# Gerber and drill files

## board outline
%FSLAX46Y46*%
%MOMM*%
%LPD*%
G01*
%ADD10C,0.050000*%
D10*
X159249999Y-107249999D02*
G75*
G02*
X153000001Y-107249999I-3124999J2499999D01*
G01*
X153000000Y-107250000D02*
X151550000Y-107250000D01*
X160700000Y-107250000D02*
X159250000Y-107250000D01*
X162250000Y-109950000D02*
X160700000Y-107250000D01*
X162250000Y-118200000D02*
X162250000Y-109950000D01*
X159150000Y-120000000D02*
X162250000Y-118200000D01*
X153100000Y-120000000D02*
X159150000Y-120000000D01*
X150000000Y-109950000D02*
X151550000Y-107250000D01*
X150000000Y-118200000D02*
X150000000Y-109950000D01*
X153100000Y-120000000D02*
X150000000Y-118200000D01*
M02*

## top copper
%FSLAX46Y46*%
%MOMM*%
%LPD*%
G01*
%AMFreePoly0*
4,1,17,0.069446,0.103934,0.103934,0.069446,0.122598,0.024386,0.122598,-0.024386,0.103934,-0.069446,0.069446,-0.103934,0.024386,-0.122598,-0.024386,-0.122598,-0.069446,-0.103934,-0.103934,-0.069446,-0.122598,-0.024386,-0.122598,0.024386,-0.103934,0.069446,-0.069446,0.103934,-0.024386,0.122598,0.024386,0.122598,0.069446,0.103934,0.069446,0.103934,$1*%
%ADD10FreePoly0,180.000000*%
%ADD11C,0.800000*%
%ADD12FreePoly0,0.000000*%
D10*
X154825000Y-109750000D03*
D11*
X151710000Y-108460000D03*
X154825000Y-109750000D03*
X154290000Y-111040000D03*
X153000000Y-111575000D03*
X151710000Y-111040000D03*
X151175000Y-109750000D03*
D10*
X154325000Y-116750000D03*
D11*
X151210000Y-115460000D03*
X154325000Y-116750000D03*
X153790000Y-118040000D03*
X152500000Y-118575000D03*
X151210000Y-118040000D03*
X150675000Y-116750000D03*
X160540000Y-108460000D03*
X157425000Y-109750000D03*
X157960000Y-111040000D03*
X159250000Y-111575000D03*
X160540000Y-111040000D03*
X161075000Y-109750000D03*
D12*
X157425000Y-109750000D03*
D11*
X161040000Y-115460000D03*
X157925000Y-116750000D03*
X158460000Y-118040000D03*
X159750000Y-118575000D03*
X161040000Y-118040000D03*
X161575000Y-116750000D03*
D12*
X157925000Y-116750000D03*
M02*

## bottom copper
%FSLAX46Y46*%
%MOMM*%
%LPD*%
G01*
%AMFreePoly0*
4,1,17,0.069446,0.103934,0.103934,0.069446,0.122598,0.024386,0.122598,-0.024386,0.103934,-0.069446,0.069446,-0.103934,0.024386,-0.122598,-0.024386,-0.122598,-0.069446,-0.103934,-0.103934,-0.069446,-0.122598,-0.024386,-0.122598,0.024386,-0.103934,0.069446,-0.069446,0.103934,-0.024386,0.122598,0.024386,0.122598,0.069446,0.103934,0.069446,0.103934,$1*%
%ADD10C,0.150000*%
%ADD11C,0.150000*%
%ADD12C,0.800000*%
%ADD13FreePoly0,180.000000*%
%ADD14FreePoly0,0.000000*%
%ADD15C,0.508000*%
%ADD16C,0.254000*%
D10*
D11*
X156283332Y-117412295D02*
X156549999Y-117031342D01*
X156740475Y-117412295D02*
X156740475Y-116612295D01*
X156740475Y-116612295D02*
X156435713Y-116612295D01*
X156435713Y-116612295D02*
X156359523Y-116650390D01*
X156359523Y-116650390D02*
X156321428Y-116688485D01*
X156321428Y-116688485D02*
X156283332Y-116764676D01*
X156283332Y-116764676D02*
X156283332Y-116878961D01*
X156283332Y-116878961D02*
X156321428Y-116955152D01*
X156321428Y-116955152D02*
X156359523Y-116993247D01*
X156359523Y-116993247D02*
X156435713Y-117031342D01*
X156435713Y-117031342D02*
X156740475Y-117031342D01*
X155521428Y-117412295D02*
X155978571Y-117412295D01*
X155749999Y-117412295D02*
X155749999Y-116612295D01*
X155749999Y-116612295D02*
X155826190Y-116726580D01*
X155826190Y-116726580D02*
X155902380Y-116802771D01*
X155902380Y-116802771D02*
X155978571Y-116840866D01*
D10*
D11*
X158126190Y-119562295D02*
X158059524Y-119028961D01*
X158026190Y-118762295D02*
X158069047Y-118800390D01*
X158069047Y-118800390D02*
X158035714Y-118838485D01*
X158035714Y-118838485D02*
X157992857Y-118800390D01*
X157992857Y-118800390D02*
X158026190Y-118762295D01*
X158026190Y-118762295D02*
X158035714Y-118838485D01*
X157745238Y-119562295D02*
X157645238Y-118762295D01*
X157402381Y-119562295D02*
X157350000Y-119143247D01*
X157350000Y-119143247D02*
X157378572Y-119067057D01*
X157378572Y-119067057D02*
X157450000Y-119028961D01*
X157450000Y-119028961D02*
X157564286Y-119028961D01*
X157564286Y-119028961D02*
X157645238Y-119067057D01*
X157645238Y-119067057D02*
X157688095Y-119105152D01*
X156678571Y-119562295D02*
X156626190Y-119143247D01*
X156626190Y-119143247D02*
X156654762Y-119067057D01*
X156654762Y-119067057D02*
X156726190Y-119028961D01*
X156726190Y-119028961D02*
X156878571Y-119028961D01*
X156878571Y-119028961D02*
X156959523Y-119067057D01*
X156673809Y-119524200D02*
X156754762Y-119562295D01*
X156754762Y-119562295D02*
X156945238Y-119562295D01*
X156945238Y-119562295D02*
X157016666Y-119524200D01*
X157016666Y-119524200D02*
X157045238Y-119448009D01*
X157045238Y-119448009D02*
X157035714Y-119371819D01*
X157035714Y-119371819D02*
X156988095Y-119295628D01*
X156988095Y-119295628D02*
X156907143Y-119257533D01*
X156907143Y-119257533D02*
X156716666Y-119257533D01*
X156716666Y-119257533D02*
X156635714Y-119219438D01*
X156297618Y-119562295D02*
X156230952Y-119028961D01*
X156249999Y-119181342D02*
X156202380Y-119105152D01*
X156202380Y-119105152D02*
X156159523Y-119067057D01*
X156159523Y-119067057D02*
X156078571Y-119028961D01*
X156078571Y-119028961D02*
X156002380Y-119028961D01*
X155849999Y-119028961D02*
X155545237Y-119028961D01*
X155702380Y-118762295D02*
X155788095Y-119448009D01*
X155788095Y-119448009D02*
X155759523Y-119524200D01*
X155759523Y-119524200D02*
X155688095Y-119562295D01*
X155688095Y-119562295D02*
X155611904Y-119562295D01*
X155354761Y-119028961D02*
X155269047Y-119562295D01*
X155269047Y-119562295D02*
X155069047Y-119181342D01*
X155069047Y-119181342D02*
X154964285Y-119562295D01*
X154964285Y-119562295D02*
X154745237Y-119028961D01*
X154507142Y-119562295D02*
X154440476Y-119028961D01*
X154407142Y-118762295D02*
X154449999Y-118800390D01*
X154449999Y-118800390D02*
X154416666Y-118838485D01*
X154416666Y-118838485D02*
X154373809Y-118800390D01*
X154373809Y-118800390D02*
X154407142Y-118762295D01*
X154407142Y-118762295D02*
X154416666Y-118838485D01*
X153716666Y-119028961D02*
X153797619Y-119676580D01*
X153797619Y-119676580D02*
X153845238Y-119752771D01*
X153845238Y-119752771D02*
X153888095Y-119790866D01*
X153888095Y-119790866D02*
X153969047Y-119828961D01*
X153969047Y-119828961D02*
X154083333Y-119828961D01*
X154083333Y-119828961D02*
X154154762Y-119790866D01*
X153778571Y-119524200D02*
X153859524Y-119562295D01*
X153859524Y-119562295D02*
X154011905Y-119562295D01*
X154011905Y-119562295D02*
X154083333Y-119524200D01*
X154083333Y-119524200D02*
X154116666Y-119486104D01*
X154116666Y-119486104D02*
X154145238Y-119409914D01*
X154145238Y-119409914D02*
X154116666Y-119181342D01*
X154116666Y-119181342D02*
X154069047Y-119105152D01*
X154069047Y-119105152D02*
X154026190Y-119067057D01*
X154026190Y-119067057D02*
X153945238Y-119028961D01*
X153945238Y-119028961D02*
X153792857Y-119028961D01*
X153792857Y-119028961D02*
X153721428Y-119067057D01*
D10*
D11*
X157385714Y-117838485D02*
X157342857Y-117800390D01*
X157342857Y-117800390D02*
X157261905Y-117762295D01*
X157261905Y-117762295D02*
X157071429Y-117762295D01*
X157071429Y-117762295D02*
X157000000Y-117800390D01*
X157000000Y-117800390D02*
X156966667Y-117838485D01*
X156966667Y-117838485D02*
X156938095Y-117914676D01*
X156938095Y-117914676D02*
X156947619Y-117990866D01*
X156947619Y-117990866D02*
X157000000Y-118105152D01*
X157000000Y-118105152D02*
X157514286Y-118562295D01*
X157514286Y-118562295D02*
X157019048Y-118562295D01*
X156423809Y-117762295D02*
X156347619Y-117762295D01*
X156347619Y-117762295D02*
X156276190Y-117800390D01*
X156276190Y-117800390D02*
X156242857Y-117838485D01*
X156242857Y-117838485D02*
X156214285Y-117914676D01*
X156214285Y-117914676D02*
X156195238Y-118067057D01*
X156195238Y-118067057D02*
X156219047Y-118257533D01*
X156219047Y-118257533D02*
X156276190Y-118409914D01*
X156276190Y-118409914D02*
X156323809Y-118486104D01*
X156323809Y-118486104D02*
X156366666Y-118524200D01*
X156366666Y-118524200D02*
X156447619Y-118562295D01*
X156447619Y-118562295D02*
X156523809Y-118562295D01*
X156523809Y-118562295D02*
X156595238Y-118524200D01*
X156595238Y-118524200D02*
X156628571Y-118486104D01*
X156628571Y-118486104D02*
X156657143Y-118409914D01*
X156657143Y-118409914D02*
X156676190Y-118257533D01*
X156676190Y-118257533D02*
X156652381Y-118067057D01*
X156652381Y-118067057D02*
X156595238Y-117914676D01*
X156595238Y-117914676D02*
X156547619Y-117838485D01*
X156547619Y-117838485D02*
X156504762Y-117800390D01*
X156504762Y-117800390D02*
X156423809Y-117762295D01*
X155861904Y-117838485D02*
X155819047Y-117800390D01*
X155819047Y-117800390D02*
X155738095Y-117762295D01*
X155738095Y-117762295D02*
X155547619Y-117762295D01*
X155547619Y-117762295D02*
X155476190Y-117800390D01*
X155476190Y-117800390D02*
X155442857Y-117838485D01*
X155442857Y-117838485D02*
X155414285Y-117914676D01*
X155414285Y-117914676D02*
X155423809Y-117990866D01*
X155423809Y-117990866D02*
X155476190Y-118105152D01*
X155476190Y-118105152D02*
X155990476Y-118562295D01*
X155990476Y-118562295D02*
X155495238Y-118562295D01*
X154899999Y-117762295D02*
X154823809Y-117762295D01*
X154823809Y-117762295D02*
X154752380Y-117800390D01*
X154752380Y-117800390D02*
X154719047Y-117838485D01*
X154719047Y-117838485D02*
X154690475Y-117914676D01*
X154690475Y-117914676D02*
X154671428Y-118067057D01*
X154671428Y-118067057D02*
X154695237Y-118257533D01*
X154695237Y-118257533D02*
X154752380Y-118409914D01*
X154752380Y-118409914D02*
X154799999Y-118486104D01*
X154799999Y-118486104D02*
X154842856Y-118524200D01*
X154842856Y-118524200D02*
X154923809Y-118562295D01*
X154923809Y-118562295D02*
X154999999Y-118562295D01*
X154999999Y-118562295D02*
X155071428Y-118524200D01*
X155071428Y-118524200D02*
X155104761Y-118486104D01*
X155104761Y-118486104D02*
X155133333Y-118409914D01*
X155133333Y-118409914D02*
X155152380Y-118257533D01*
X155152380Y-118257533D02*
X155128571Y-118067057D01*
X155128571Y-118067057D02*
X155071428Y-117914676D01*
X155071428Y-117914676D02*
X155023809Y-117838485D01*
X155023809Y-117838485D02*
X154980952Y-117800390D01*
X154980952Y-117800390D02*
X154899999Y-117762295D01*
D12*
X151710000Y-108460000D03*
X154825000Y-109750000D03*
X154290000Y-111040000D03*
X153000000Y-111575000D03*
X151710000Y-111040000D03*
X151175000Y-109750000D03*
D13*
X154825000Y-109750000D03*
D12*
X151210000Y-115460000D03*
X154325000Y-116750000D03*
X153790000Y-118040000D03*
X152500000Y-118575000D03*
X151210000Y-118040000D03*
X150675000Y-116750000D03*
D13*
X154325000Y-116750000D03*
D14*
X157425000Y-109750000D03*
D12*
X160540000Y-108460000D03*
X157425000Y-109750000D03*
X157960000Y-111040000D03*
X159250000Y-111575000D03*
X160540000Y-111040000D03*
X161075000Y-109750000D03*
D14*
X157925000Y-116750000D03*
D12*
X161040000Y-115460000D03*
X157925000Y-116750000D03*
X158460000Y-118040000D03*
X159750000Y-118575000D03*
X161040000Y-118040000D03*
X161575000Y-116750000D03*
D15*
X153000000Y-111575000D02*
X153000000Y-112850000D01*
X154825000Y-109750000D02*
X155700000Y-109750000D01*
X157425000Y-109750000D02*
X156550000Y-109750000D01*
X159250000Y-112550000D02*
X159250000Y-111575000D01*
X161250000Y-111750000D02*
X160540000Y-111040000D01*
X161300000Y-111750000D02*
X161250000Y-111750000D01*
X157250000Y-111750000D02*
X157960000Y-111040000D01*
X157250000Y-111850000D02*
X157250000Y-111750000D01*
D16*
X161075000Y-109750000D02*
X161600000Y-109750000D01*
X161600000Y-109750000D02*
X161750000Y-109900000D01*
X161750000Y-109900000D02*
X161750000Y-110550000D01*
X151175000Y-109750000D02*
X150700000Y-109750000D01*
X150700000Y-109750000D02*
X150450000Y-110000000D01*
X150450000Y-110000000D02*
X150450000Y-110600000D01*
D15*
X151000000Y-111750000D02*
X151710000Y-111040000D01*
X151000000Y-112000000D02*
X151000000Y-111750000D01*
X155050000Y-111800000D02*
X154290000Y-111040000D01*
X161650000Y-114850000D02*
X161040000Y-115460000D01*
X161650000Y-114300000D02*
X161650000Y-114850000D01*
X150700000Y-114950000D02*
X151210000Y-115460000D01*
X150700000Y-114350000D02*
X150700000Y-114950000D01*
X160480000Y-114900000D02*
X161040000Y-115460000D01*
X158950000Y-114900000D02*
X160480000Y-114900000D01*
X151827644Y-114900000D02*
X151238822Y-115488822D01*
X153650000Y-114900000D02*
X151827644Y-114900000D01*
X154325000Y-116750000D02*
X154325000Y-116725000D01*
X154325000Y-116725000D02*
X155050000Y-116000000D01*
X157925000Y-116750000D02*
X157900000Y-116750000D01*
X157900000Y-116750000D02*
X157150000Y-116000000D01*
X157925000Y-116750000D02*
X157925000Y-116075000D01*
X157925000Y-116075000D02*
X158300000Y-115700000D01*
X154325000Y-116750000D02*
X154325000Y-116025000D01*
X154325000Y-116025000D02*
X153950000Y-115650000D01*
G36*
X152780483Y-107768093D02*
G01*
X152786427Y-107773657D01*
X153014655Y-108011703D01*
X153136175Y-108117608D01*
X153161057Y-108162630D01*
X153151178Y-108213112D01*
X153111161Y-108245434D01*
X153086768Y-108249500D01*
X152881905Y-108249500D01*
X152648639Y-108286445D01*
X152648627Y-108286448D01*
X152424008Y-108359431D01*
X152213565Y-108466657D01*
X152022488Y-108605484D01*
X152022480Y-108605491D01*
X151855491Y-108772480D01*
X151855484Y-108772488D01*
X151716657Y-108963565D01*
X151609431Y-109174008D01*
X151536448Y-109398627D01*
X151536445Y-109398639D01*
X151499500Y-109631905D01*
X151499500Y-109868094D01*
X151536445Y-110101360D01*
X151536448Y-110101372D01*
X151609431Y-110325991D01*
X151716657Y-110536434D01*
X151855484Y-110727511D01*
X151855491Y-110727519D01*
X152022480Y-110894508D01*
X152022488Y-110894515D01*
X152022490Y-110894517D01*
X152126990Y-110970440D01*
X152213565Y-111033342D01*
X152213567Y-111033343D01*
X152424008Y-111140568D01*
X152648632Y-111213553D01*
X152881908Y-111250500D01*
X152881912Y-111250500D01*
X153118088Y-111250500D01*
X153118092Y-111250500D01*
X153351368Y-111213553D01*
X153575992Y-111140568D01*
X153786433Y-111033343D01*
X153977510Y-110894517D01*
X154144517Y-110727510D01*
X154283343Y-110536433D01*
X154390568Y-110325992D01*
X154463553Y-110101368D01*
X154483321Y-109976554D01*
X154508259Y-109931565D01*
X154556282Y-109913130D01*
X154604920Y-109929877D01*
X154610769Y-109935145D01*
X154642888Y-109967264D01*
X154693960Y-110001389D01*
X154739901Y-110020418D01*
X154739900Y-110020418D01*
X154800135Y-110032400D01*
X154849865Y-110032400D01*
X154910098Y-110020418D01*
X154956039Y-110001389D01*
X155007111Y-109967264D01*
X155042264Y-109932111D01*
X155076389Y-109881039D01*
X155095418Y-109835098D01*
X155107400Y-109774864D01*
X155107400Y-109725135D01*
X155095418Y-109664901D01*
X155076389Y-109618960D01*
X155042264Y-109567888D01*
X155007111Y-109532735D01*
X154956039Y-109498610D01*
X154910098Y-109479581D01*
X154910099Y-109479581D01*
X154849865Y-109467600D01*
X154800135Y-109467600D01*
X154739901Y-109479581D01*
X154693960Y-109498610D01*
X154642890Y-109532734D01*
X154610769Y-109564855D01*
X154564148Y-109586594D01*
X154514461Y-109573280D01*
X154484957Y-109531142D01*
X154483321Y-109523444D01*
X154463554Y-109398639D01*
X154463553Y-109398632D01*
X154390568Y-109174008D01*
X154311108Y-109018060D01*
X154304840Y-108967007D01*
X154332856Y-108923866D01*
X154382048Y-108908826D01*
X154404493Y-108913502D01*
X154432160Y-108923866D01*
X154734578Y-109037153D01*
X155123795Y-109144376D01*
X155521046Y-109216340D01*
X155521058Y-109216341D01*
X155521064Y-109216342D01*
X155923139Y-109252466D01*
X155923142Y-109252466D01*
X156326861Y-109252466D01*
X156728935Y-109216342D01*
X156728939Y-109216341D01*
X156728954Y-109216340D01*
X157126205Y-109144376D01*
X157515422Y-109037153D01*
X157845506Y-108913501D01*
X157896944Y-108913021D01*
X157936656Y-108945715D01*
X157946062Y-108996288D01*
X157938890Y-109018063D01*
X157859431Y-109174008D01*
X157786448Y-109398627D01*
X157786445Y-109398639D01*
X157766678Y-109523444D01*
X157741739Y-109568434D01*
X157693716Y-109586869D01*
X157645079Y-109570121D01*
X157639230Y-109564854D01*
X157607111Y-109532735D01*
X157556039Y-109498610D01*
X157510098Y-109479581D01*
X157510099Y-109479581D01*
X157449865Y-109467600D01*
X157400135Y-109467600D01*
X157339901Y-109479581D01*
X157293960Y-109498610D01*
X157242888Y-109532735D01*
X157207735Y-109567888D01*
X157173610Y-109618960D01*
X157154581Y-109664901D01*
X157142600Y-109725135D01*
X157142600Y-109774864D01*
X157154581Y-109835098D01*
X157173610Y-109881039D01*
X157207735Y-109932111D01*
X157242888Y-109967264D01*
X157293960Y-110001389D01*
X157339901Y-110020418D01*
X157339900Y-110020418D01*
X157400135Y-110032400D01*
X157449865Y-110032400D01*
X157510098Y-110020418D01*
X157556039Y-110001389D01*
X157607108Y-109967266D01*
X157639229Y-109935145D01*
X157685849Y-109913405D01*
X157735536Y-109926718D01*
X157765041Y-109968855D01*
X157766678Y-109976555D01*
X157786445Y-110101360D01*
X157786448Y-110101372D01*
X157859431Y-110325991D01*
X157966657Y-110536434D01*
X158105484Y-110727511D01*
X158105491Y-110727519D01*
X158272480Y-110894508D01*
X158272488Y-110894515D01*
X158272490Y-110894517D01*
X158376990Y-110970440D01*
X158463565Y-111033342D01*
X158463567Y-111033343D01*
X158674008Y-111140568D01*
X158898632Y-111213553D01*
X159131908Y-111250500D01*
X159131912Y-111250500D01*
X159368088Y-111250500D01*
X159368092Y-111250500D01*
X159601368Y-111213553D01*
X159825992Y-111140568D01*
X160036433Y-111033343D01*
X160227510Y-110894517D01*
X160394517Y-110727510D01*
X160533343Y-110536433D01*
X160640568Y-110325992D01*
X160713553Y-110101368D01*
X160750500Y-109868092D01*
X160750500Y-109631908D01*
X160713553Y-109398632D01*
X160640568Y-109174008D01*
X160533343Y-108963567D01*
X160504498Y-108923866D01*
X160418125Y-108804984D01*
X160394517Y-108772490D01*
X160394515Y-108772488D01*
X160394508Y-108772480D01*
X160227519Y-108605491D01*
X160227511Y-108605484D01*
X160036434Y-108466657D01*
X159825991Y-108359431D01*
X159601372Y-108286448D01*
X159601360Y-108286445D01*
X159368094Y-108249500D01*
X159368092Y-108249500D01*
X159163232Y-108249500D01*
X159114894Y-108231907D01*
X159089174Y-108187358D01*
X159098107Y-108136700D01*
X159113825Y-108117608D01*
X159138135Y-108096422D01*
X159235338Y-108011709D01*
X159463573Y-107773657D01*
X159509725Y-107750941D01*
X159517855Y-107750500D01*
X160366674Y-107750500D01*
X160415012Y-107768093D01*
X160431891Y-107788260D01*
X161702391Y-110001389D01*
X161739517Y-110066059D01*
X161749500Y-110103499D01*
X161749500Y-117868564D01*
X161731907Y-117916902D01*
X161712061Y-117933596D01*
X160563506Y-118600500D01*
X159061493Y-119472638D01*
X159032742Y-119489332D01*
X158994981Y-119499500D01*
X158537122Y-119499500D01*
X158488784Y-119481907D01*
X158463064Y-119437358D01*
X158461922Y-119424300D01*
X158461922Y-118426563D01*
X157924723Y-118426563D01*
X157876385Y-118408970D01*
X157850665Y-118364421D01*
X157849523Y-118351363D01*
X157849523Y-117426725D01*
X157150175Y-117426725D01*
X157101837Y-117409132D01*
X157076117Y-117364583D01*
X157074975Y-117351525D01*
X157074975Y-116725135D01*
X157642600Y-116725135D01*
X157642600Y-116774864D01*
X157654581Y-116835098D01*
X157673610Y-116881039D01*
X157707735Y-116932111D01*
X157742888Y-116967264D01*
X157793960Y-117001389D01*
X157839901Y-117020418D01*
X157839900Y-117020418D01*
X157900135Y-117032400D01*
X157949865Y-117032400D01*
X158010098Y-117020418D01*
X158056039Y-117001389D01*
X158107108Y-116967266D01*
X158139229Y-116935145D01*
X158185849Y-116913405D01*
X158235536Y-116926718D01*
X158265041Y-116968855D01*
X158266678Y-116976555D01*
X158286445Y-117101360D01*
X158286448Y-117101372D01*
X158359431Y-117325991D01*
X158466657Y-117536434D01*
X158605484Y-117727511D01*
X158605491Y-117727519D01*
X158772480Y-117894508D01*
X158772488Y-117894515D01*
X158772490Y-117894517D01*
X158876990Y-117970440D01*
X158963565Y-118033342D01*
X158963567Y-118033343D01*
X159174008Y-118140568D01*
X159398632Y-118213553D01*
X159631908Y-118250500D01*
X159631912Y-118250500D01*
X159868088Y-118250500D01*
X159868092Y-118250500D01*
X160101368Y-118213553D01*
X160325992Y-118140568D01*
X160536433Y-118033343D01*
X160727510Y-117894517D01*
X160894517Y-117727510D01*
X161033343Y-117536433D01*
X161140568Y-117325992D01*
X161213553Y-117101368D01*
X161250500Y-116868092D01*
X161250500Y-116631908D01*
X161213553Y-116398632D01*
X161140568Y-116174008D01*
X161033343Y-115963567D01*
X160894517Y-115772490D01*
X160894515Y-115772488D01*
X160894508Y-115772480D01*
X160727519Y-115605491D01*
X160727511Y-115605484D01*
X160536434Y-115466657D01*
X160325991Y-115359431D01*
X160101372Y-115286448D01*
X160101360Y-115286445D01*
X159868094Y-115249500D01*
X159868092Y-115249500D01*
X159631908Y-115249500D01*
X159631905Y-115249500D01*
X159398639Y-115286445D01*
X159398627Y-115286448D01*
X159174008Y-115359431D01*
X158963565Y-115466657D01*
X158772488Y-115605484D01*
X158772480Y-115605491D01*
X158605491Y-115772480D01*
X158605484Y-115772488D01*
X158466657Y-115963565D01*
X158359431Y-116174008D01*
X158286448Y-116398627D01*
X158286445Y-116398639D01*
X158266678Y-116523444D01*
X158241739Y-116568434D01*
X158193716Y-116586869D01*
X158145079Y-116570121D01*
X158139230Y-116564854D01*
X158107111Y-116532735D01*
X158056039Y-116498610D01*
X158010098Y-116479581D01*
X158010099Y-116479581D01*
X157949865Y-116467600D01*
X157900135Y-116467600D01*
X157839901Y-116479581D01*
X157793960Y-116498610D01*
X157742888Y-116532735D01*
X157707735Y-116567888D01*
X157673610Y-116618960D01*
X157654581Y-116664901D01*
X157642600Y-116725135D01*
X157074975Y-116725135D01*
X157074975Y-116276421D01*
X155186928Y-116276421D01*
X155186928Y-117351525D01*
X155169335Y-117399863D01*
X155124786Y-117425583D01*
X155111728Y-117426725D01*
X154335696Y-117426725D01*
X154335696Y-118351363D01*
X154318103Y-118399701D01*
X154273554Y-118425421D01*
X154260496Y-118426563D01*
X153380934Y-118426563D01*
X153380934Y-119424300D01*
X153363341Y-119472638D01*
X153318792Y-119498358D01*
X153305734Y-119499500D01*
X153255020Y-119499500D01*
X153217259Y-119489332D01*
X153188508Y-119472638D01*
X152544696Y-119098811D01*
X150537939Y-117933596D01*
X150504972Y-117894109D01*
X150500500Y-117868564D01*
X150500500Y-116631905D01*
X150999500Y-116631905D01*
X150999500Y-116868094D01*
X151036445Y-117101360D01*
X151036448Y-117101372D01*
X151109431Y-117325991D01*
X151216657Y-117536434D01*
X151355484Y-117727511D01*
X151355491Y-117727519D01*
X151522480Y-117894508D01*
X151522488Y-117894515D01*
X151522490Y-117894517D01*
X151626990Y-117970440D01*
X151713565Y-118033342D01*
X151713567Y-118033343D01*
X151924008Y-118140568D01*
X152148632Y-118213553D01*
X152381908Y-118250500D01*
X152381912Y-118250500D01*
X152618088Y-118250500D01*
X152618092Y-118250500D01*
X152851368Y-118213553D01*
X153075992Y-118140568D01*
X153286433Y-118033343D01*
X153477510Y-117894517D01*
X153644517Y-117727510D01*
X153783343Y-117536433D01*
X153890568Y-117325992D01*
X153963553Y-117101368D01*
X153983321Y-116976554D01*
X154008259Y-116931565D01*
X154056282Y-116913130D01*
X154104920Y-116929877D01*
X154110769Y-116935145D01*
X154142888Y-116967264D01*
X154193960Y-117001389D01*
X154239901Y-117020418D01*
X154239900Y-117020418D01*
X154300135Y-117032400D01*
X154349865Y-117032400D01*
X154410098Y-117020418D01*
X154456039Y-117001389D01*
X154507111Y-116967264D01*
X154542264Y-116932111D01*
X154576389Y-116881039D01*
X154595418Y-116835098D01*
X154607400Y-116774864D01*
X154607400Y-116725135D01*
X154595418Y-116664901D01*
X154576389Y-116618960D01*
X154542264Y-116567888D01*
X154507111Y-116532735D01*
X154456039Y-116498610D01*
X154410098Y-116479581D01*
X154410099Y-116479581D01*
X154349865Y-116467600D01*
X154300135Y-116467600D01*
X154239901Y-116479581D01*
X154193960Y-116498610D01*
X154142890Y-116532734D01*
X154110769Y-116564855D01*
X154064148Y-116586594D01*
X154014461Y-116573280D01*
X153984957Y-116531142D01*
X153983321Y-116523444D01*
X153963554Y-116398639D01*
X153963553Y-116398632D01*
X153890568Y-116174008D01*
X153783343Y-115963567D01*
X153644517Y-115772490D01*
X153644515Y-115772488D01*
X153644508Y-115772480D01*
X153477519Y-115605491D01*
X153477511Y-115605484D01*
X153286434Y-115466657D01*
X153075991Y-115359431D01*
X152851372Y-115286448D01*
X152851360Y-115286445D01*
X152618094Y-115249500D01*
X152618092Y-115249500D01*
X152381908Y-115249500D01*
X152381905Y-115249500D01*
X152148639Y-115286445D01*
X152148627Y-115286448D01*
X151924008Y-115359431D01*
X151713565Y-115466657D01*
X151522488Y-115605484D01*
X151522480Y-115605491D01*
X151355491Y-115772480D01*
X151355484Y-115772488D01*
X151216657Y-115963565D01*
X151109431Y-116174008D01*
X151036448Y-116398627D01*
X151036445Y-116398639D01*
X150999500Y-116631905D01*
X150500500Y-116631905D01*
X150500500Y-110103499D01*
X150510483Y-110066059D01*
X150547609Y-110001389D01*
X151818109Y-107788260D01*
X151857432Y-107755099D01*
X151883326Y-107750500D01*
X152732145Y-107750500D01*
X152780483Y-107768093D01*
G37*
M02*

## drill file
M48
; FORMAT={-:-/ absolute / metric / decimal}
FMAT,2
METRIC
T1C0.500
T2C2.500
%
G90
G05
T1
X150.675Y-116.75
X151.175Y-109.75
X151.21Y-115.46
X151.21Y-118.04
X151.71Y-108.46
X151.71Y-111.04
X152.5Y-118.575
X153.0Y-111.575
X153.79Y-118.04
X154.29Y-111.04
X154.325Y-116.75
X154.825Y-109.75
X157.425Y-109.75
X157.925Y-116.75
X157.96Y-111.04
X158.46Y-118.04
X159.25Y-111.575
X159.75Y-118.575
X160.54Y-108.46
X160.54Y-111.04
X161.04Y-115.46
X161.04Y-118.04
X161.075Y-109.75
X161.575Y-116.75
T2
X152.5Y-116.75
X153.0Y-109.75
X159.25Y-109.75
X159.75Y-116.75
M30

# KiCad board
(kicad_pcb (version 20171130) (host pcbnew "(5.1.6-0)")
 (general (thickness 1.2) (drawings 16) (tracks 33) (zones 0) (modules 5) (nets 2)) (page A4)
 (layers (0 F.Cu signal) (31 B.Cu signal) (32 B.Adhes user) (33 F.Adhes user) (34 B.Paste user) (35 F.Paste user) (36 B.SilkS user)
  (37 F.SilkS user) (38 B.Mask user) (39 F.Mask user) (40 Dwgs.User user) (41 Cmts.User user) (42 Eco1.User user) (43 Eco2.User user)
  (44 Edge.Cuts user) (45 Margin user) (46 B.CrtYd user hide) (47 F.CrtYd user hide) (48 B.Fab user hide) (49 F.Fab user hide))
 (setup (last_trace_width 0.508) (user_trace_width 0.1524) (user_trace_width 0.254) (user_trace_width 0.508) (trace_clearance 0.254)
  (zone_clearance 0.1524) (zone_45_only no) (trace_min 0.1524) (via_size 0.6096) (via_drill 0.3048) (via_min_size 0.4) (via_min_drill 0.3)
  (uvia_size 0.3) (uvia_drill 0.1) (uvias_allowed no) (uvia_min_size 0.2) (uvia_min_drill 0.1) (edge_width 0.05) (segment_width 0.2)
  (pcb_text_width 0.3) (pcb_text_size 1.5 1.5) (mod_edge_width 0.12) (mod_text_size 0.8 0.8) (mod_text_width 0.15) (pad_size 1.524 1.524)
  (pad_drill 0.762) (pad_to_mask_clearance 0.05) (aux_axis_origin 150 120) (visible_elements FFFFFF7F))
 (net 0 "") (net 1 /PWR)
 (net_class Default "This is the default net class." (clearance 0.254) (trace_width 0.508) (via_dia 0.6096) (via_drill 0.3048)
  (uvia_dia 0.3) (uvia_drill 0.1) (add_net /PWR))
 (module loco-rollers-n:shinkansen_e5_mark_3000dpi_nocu (layer F.Cu) (at 156.95 113.75)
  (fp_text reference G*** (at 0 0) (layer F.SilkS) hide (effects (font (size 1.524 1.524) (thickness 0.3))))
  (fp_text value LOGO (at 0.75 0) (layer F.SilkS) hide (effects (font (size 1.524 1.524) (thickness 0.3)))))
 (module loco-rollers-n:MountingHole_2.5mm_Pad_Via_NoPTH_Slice (layer B.Cu) (at 153 109.75 180)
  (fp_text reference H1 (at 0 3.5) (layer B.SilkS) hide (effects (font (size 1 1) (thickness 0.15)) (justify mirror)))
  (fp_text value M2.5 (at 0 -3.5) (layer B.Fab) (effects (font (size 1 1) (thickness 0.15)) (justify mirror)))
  (pad 1 smd custom (at -1.825 0 180) (size 0.25 0.25) (layers F.Cu F.Mask) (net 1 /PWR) (solder_mask_margin 0.25) (zone_connect 0)
   (options (clearance outline) (anchor circle)) (primitives))
  (pad "" np_thru_hole circle (at 0 0 180) (size 2.5 2.5) (drill 2.5) (layers *.Cu *.Mask) (solder_mask_margin 0.25))
  (pad 1 thru_hole circle (at 1.29 1.29 180) (size 0.8 0.8) (drill 0.5) (layers *.Cu *.Mask) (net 1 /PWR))
  (pad 1 thru_hole circle (at -1.825 0 180) (size 0.8 0.8) (drill 0.5) (layers *.Cu *.Mask) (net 1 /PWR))
  (pad 1 thru_hole circle (at -1.29 -1.29 180) (size 0.8 0.8) (drill 0.5) (layers *.Cu *.Mask) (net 1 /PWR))
  (pad 1 thru_hole circle (at 0 -1.825 180) (size 0.8 0.8) (drill 0.5) (layers *.Cu *.Mask) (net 1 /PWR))
  (pad 1 thru_hole circle (at 1.29 -1.29 180) (size 0.8 0.8) (drill 0.5) (layers *.Cu *.Mask) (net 1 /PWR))
  (pad 1 thru_hole circle (at 1.825 0 180) (size 0.8 0.8) (drill 0.5) (layers *.Cu *.Mask) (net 1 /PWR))
  (pad 1 smd custom (at -1.825 0 180) (size 0.25 0.25) (layers B.Cu B.Mask) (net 1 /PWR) (solder_mask_margin 0.25) (zone_connect 0)
   (options (clearance outline) (anchor circle)) (primitives)))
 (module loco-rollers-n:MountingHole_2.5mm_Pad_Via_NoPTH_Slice (layer B.Cu) (at 152.5 116.75 180)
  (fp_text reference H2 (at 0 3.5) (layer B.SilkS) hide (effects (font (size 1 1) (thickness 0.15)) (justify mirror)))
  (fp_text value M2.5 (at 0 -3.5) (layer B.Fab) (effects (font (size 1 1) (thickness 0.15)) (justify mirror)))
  (pad 1 smd custom (at -1.825 0 180) (size 0.25 0.25) (layers F.Cu F.Mask) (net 1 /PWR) (solder_mask_margin 0.25) (zone_connect 0)
   (options (clearance outline) (anchor circle)) (primitives))
  (pad "" np_thru_hole circle (at 0 0 180) (size 2.5 2.5) (drill 2.5) (layers *.Cu *.Mask) (solder_mask_margin 0.25))
  (pad 1 thru_hole circle (at 1.29 1.29 180) (size 0.8 0.8) (drill 0.5) (layers *.Cu *.Mask) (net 1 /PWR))
  (pad 1 thru_hole circle (at -1.825 0 180) (size 0.8 0.8) (drill 0.5) (layers *.Cu *.Mask) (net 1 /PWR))
  (pad 1 thru_hole circle (at -1.29 -1.29 180) (size 0.8 0.8) (drill 0.5) (layers *.Cu *.Mask) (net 1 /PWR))
  (pad 1 thru_hole circle (at 0 -1.825 180) (size 0.8 0.8) (drill 0.5) (layers *.Cu *.Mask) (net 1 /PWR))
  (pad 1 thru_hole circle (at 1.29 -1.29 180) (size 0.8 0.8) (drill 0.5) (layers *.Cu *.Mask) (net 1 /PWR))
  (pad 1 thru_hole circle (at 1.825 0 180) (size 0.8 0.8) (drill 0.5) (layers *.Cu *.Mask) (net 1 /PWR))
  (pad 1 smd custom (at -1.825 0 180) (size 0.25 0.25) (layers B.Cu B.Mask) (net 1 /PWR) (solder_mask_margin 0.25) (zone_connect 0)
   (options (clearance outline) (anchor circle)) (primitives)))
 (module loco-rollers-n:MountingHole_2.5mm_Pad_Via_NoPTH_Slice (layer F.Cu) (at 159.25 109.75)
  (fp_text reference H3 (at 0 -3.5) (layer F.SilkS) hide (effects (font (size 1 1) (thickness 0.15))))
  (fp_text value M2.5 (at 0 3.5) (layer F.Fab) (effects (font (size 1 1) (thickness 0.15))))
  (pad 1 smd custom (at -1.825 0) (size 0.25 0.25) (layers B.Cu B.Mask) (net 1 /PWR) (solder_mask_margin 0.25) (zone_connect 0)
   (options (clearance outline) (anchor circle)) (primitives))
  (pad "" np_thru_hole circle (at 0 0) (size 2.5 2.5) (drill 2.5) (layers *.Cu *.Mask) (solder_mask_margin 0.25))
  (pad 1 thru_hole circle (at 1.29 -1.29) (size 0.8 0.8) (drill 0.5) (layers *.Cu *.Mask) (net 1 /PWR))
  (pad 1 thru_hole circle (at -1.825 0) (size 0.8 0.8) (drill 0.5) (layers *.Cu *.Mask) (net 1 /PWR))
  (pad 1 thru_hole circle (at -1.29 1.29) (size 0.8 0.8) (drill 0.5) (layers *.Cu *.Mask) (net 1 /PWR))
  (pad 1 thru_hole circle (at 0 1.825) (size 0.8 0.8) (drill 0.5) (layers *.Cu *.Mask) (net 1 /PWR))
  (pad 1 thru_hole circle (at 1.29 1.29) (size 0.8 0.8) (drill 0.5) (layers *.Cu *.Mask) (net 1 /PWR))
  (pad 1 thru_hole circle (at 1.825 0) (size 0.8 0.8) (drill 0.5) (layers *.Cu *.Mask) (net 1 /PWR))
  (pad 1 smd custom (at -1.825 0) (size 0.25 0.25) (layers F.Cu F.Mask) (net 1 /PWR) (solder_mask_margin 0.25) (zone_connect 0)
   (options (clearance outline) (anchor circle)) (primitives)))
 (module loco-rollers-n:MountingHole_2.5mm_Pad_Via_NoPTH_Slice (layer F.Cu) (at 159.75 116.75)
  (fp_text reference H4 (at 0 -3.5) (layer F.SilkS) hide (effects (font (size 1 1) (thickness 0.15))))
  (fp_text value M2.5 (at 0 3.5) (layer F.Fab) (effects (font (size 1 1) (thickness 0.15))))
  (pad 1 smd custom (at -1.825 0) (size 0.25 0.25) (layers B.Cu B.Mask) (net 1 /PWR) (solder_mask_margin 0.25) (zone_connect 0)
   (options (clearance outline) (anchor circle)) (primitives))
  (pad "" np_thru_hole circle (at 0 0) (size 2.5 2.5) (drill 2.5) (layers *.Cu *.Mask) (solder_mask_margin 0.25))
  (pad 1 thru_hole circle (at 1.29 -1.29) (size 0.8 0.8) (drill 0.5) (layers *.Cu *.Mask) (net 1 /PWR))
  (pad 1 thru_hole circle (at -1.825 0) (size 0.8 0.8) (drill 0.5) (layers *.Cu *.Mask) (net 1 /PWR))
  (pad 1 thru_hole circle (at -1.29 1.29) (size 0.8 0.8) (drill 0.5) (layers *.Cu *.Mask) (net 1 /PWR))
  (pad 1 thru_hole circle (at 0 1.825) (size 0.8 0.8) (drill 0.5) (layers *.Cu *.Mask) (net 1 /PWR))
  (pad 1 thru_hole circle (at 1.29 1.29) (size 0.8 0.8) (drill 0.5) (layers *.Cu *.Mask) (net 1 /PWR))
  (pad 1 thru_hole circle (at 1.825 0) (size 0.8 0.8) (drill 0.5) (layers *.Cu *.Mask) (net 1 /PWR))
  (pad 1 smd custom (at -1.825 0) (size 0.25 0.25) (layers F.Cu F.Mask) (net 1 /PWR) (solder_mask_margin 0.25) (zone_connect 0)
   (options (clearance outline) (anchor circle)) (primitives)))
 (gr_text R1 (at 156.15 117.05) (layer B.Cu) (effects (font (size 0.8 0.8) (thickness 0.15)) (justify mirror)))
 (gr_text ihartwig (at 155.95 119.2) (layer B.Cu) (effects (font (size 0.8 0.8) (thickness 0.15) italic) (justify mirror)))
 (gr_arc (start 156.125 104.75) (end 153.000001 107.249999) (angle -102.6803835) (layer Edge.Cuts) (width 0.05))
 (gr_line (start 153 107.25) (end 151.55 107.25) (layer Edge.Cuts) (width 0.05))
 (gr_line (start 160.7 107.25) (end 159.25 107.25) (layer Edge.Cuts) (width 0.05))
 (gr_line (start 162.25 109.95) (end 160.7 107.25) (layer Edge.Cuts) (width 0.05))
 (gr_line (start 162.25 118.2) (end 162.25 109.95) (layer Edge.Cuts) (width 0.05))
 (gr_line (start 159.15 120) (end 162.25 118.2) (layer Edge.Cuts) (width 0.05))
 (gr_line (start 153.1 120) (end 159.15 120) (layer Edge.Cuts) (width 0.05))
 (gr_line (start 150 109.95) (end 151.55 107.25) (layer Edge.Cuts) (width 0.05))
 (gr_line (start 150 118.2) (end 150 109.95) (layer Edge.Cuts) (width 0.05))
 (gr_line (start 153.1 120) (end 150 118.2) (layer Edge.Cuts) (width 0.05))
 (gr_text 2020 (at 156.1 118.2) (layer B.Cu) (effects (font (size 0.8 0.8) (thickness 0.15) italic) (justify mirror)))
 (segment (start 153 111.575) (end 153 112.85) (width 0.508) (layer B.Cu) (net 1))
 (segment (start 154.825 109.75) (end 155.7 109.75) (width 0.508) (layer B.Cu) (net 1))
 (segment (start 157.425 109.75) (end 156.55 109.75) (width 0.508) (layer B.Cu) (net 1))
 (segment (start 159.25 112.55) (end 159.25 111.575) (width 0.508) (layer B.Cu) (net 1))
 (segment (start 161.25 111.75) (end 160.54 111.04) (width 0.508) (layer B.Cu) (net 1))
 (segment (start 161.3 111.75) (end 161.25 111.75) (width 0.508) (layer B.Cu) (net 1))
 (segment (start 157.25 111.75) (end 157.96 111.04) (width 0.508) (layer B.Cu) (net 1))
 (segment (start 157.25 111.85) (end 157.25 111.75) (width 0.508) (layer B.Cu) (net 1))
 (segment (start 161.075 109.75) (end 161.6 109.75) (width 0.254) (layer B.Cu) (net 1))
 (segment (start 161.6 109.75) (end 161.75 109.9) (width 0.254) (layer B.Cu) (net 1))
 (segment (start 161.75 109.9) (end 161.75 110.55) (width 0.254) (layer B.Cu) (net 1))
 (segment (start 151.175 109.75) (end 150.7 109.75) (width 0.254) (layer B.Cu) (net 1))
 (segment (start 150.7 109.75) (end 150.45 110) (width 0.254) (layer B.Cu) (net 1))
 (segment (start 150.45 110) (end 150.45 110.6) (width 0.254) (layer B.Cu) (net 1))
 (segment (start 151 111.75) (end 151.71 111.04) (width 0.508) (layer B.Cu) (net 1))
 (segment (start 151 112) (end 151 111.75) (width 0.508) (layer B.Cu) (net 1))
 (segment (start 155.05 111.8) (end 154.29 111.04) (width 0.508) (layer B.Cu) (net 1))
 (segment (start 161.65 114.85) (end 161.04 115.46) (width 0.508) (layer B.Cu) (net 1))
 (segment (start 161.65 114.3) (end 161.65 114.85) (width 0.508) (layer B.Cu) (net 1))
 (segment (start 150.7 114.95) (end 151.21 115.46) (width 0.508) (layer B.Cu) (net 1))
 (segment (start 150.7 114.35) (end 150.7 114.95) (width 0.508) (layer B.Cu) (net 1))
 (segment (start 160.48 114.9) (end 161.04 115.46) (width 0.508) (layer B.Cu) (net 1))
 (segment (start 158.95 114.9) (end 160.48 114.9) (width 0.508) (layer B.Cu) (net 1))
 (segment (start 151.827644 114.9) (end 151.238822 115.488822) (width 0.508) (layer B.Cu) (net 1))
 (segment (start 153.65 114.9) (end 151.827644 114.9) (width 0.508) (layer B.Cu) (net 1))
 (segment (start 154.325 116.75) (end 154.325 116.725) (width 0.508) (layer B.Cu) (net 1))
 (segment (start 154.325 116.725) (end 155.05 116) (width 0.508) (layer B.Cu) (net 1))
 (segment (start 157.925 116.75) (end 157.9 116.75) (width 0.508) (layer B.Cu) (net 1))
 (segment (start 157.9 116.75) (end 157.15 116) (width 0.508) (layer B.Cu) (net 1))
 (segment (start 157.925 116.75) (end 157.925 116.075) (width 0.508) (layer B.Cu) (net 1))
 (segment (start 157.925 116.075) (end 158.3 115.7) (width 0.508) (layer B.Cu) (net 1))
 (segment (start 154.325 116.75) (end 154.325 116.025) (width 0.508) (layer B.Cu) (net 1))
 (segment (start 154.325 116.025) (end 153.95 115.65) (width 0.508) (layer B.Cu) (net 1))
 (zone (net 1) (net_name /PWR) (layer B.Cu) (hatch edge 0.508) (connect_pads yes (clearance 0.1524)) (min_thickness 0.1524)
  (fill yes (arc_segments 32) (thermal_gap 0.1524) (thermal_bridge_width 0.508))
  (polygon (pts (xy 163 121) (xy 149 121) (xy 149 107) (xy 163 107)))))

